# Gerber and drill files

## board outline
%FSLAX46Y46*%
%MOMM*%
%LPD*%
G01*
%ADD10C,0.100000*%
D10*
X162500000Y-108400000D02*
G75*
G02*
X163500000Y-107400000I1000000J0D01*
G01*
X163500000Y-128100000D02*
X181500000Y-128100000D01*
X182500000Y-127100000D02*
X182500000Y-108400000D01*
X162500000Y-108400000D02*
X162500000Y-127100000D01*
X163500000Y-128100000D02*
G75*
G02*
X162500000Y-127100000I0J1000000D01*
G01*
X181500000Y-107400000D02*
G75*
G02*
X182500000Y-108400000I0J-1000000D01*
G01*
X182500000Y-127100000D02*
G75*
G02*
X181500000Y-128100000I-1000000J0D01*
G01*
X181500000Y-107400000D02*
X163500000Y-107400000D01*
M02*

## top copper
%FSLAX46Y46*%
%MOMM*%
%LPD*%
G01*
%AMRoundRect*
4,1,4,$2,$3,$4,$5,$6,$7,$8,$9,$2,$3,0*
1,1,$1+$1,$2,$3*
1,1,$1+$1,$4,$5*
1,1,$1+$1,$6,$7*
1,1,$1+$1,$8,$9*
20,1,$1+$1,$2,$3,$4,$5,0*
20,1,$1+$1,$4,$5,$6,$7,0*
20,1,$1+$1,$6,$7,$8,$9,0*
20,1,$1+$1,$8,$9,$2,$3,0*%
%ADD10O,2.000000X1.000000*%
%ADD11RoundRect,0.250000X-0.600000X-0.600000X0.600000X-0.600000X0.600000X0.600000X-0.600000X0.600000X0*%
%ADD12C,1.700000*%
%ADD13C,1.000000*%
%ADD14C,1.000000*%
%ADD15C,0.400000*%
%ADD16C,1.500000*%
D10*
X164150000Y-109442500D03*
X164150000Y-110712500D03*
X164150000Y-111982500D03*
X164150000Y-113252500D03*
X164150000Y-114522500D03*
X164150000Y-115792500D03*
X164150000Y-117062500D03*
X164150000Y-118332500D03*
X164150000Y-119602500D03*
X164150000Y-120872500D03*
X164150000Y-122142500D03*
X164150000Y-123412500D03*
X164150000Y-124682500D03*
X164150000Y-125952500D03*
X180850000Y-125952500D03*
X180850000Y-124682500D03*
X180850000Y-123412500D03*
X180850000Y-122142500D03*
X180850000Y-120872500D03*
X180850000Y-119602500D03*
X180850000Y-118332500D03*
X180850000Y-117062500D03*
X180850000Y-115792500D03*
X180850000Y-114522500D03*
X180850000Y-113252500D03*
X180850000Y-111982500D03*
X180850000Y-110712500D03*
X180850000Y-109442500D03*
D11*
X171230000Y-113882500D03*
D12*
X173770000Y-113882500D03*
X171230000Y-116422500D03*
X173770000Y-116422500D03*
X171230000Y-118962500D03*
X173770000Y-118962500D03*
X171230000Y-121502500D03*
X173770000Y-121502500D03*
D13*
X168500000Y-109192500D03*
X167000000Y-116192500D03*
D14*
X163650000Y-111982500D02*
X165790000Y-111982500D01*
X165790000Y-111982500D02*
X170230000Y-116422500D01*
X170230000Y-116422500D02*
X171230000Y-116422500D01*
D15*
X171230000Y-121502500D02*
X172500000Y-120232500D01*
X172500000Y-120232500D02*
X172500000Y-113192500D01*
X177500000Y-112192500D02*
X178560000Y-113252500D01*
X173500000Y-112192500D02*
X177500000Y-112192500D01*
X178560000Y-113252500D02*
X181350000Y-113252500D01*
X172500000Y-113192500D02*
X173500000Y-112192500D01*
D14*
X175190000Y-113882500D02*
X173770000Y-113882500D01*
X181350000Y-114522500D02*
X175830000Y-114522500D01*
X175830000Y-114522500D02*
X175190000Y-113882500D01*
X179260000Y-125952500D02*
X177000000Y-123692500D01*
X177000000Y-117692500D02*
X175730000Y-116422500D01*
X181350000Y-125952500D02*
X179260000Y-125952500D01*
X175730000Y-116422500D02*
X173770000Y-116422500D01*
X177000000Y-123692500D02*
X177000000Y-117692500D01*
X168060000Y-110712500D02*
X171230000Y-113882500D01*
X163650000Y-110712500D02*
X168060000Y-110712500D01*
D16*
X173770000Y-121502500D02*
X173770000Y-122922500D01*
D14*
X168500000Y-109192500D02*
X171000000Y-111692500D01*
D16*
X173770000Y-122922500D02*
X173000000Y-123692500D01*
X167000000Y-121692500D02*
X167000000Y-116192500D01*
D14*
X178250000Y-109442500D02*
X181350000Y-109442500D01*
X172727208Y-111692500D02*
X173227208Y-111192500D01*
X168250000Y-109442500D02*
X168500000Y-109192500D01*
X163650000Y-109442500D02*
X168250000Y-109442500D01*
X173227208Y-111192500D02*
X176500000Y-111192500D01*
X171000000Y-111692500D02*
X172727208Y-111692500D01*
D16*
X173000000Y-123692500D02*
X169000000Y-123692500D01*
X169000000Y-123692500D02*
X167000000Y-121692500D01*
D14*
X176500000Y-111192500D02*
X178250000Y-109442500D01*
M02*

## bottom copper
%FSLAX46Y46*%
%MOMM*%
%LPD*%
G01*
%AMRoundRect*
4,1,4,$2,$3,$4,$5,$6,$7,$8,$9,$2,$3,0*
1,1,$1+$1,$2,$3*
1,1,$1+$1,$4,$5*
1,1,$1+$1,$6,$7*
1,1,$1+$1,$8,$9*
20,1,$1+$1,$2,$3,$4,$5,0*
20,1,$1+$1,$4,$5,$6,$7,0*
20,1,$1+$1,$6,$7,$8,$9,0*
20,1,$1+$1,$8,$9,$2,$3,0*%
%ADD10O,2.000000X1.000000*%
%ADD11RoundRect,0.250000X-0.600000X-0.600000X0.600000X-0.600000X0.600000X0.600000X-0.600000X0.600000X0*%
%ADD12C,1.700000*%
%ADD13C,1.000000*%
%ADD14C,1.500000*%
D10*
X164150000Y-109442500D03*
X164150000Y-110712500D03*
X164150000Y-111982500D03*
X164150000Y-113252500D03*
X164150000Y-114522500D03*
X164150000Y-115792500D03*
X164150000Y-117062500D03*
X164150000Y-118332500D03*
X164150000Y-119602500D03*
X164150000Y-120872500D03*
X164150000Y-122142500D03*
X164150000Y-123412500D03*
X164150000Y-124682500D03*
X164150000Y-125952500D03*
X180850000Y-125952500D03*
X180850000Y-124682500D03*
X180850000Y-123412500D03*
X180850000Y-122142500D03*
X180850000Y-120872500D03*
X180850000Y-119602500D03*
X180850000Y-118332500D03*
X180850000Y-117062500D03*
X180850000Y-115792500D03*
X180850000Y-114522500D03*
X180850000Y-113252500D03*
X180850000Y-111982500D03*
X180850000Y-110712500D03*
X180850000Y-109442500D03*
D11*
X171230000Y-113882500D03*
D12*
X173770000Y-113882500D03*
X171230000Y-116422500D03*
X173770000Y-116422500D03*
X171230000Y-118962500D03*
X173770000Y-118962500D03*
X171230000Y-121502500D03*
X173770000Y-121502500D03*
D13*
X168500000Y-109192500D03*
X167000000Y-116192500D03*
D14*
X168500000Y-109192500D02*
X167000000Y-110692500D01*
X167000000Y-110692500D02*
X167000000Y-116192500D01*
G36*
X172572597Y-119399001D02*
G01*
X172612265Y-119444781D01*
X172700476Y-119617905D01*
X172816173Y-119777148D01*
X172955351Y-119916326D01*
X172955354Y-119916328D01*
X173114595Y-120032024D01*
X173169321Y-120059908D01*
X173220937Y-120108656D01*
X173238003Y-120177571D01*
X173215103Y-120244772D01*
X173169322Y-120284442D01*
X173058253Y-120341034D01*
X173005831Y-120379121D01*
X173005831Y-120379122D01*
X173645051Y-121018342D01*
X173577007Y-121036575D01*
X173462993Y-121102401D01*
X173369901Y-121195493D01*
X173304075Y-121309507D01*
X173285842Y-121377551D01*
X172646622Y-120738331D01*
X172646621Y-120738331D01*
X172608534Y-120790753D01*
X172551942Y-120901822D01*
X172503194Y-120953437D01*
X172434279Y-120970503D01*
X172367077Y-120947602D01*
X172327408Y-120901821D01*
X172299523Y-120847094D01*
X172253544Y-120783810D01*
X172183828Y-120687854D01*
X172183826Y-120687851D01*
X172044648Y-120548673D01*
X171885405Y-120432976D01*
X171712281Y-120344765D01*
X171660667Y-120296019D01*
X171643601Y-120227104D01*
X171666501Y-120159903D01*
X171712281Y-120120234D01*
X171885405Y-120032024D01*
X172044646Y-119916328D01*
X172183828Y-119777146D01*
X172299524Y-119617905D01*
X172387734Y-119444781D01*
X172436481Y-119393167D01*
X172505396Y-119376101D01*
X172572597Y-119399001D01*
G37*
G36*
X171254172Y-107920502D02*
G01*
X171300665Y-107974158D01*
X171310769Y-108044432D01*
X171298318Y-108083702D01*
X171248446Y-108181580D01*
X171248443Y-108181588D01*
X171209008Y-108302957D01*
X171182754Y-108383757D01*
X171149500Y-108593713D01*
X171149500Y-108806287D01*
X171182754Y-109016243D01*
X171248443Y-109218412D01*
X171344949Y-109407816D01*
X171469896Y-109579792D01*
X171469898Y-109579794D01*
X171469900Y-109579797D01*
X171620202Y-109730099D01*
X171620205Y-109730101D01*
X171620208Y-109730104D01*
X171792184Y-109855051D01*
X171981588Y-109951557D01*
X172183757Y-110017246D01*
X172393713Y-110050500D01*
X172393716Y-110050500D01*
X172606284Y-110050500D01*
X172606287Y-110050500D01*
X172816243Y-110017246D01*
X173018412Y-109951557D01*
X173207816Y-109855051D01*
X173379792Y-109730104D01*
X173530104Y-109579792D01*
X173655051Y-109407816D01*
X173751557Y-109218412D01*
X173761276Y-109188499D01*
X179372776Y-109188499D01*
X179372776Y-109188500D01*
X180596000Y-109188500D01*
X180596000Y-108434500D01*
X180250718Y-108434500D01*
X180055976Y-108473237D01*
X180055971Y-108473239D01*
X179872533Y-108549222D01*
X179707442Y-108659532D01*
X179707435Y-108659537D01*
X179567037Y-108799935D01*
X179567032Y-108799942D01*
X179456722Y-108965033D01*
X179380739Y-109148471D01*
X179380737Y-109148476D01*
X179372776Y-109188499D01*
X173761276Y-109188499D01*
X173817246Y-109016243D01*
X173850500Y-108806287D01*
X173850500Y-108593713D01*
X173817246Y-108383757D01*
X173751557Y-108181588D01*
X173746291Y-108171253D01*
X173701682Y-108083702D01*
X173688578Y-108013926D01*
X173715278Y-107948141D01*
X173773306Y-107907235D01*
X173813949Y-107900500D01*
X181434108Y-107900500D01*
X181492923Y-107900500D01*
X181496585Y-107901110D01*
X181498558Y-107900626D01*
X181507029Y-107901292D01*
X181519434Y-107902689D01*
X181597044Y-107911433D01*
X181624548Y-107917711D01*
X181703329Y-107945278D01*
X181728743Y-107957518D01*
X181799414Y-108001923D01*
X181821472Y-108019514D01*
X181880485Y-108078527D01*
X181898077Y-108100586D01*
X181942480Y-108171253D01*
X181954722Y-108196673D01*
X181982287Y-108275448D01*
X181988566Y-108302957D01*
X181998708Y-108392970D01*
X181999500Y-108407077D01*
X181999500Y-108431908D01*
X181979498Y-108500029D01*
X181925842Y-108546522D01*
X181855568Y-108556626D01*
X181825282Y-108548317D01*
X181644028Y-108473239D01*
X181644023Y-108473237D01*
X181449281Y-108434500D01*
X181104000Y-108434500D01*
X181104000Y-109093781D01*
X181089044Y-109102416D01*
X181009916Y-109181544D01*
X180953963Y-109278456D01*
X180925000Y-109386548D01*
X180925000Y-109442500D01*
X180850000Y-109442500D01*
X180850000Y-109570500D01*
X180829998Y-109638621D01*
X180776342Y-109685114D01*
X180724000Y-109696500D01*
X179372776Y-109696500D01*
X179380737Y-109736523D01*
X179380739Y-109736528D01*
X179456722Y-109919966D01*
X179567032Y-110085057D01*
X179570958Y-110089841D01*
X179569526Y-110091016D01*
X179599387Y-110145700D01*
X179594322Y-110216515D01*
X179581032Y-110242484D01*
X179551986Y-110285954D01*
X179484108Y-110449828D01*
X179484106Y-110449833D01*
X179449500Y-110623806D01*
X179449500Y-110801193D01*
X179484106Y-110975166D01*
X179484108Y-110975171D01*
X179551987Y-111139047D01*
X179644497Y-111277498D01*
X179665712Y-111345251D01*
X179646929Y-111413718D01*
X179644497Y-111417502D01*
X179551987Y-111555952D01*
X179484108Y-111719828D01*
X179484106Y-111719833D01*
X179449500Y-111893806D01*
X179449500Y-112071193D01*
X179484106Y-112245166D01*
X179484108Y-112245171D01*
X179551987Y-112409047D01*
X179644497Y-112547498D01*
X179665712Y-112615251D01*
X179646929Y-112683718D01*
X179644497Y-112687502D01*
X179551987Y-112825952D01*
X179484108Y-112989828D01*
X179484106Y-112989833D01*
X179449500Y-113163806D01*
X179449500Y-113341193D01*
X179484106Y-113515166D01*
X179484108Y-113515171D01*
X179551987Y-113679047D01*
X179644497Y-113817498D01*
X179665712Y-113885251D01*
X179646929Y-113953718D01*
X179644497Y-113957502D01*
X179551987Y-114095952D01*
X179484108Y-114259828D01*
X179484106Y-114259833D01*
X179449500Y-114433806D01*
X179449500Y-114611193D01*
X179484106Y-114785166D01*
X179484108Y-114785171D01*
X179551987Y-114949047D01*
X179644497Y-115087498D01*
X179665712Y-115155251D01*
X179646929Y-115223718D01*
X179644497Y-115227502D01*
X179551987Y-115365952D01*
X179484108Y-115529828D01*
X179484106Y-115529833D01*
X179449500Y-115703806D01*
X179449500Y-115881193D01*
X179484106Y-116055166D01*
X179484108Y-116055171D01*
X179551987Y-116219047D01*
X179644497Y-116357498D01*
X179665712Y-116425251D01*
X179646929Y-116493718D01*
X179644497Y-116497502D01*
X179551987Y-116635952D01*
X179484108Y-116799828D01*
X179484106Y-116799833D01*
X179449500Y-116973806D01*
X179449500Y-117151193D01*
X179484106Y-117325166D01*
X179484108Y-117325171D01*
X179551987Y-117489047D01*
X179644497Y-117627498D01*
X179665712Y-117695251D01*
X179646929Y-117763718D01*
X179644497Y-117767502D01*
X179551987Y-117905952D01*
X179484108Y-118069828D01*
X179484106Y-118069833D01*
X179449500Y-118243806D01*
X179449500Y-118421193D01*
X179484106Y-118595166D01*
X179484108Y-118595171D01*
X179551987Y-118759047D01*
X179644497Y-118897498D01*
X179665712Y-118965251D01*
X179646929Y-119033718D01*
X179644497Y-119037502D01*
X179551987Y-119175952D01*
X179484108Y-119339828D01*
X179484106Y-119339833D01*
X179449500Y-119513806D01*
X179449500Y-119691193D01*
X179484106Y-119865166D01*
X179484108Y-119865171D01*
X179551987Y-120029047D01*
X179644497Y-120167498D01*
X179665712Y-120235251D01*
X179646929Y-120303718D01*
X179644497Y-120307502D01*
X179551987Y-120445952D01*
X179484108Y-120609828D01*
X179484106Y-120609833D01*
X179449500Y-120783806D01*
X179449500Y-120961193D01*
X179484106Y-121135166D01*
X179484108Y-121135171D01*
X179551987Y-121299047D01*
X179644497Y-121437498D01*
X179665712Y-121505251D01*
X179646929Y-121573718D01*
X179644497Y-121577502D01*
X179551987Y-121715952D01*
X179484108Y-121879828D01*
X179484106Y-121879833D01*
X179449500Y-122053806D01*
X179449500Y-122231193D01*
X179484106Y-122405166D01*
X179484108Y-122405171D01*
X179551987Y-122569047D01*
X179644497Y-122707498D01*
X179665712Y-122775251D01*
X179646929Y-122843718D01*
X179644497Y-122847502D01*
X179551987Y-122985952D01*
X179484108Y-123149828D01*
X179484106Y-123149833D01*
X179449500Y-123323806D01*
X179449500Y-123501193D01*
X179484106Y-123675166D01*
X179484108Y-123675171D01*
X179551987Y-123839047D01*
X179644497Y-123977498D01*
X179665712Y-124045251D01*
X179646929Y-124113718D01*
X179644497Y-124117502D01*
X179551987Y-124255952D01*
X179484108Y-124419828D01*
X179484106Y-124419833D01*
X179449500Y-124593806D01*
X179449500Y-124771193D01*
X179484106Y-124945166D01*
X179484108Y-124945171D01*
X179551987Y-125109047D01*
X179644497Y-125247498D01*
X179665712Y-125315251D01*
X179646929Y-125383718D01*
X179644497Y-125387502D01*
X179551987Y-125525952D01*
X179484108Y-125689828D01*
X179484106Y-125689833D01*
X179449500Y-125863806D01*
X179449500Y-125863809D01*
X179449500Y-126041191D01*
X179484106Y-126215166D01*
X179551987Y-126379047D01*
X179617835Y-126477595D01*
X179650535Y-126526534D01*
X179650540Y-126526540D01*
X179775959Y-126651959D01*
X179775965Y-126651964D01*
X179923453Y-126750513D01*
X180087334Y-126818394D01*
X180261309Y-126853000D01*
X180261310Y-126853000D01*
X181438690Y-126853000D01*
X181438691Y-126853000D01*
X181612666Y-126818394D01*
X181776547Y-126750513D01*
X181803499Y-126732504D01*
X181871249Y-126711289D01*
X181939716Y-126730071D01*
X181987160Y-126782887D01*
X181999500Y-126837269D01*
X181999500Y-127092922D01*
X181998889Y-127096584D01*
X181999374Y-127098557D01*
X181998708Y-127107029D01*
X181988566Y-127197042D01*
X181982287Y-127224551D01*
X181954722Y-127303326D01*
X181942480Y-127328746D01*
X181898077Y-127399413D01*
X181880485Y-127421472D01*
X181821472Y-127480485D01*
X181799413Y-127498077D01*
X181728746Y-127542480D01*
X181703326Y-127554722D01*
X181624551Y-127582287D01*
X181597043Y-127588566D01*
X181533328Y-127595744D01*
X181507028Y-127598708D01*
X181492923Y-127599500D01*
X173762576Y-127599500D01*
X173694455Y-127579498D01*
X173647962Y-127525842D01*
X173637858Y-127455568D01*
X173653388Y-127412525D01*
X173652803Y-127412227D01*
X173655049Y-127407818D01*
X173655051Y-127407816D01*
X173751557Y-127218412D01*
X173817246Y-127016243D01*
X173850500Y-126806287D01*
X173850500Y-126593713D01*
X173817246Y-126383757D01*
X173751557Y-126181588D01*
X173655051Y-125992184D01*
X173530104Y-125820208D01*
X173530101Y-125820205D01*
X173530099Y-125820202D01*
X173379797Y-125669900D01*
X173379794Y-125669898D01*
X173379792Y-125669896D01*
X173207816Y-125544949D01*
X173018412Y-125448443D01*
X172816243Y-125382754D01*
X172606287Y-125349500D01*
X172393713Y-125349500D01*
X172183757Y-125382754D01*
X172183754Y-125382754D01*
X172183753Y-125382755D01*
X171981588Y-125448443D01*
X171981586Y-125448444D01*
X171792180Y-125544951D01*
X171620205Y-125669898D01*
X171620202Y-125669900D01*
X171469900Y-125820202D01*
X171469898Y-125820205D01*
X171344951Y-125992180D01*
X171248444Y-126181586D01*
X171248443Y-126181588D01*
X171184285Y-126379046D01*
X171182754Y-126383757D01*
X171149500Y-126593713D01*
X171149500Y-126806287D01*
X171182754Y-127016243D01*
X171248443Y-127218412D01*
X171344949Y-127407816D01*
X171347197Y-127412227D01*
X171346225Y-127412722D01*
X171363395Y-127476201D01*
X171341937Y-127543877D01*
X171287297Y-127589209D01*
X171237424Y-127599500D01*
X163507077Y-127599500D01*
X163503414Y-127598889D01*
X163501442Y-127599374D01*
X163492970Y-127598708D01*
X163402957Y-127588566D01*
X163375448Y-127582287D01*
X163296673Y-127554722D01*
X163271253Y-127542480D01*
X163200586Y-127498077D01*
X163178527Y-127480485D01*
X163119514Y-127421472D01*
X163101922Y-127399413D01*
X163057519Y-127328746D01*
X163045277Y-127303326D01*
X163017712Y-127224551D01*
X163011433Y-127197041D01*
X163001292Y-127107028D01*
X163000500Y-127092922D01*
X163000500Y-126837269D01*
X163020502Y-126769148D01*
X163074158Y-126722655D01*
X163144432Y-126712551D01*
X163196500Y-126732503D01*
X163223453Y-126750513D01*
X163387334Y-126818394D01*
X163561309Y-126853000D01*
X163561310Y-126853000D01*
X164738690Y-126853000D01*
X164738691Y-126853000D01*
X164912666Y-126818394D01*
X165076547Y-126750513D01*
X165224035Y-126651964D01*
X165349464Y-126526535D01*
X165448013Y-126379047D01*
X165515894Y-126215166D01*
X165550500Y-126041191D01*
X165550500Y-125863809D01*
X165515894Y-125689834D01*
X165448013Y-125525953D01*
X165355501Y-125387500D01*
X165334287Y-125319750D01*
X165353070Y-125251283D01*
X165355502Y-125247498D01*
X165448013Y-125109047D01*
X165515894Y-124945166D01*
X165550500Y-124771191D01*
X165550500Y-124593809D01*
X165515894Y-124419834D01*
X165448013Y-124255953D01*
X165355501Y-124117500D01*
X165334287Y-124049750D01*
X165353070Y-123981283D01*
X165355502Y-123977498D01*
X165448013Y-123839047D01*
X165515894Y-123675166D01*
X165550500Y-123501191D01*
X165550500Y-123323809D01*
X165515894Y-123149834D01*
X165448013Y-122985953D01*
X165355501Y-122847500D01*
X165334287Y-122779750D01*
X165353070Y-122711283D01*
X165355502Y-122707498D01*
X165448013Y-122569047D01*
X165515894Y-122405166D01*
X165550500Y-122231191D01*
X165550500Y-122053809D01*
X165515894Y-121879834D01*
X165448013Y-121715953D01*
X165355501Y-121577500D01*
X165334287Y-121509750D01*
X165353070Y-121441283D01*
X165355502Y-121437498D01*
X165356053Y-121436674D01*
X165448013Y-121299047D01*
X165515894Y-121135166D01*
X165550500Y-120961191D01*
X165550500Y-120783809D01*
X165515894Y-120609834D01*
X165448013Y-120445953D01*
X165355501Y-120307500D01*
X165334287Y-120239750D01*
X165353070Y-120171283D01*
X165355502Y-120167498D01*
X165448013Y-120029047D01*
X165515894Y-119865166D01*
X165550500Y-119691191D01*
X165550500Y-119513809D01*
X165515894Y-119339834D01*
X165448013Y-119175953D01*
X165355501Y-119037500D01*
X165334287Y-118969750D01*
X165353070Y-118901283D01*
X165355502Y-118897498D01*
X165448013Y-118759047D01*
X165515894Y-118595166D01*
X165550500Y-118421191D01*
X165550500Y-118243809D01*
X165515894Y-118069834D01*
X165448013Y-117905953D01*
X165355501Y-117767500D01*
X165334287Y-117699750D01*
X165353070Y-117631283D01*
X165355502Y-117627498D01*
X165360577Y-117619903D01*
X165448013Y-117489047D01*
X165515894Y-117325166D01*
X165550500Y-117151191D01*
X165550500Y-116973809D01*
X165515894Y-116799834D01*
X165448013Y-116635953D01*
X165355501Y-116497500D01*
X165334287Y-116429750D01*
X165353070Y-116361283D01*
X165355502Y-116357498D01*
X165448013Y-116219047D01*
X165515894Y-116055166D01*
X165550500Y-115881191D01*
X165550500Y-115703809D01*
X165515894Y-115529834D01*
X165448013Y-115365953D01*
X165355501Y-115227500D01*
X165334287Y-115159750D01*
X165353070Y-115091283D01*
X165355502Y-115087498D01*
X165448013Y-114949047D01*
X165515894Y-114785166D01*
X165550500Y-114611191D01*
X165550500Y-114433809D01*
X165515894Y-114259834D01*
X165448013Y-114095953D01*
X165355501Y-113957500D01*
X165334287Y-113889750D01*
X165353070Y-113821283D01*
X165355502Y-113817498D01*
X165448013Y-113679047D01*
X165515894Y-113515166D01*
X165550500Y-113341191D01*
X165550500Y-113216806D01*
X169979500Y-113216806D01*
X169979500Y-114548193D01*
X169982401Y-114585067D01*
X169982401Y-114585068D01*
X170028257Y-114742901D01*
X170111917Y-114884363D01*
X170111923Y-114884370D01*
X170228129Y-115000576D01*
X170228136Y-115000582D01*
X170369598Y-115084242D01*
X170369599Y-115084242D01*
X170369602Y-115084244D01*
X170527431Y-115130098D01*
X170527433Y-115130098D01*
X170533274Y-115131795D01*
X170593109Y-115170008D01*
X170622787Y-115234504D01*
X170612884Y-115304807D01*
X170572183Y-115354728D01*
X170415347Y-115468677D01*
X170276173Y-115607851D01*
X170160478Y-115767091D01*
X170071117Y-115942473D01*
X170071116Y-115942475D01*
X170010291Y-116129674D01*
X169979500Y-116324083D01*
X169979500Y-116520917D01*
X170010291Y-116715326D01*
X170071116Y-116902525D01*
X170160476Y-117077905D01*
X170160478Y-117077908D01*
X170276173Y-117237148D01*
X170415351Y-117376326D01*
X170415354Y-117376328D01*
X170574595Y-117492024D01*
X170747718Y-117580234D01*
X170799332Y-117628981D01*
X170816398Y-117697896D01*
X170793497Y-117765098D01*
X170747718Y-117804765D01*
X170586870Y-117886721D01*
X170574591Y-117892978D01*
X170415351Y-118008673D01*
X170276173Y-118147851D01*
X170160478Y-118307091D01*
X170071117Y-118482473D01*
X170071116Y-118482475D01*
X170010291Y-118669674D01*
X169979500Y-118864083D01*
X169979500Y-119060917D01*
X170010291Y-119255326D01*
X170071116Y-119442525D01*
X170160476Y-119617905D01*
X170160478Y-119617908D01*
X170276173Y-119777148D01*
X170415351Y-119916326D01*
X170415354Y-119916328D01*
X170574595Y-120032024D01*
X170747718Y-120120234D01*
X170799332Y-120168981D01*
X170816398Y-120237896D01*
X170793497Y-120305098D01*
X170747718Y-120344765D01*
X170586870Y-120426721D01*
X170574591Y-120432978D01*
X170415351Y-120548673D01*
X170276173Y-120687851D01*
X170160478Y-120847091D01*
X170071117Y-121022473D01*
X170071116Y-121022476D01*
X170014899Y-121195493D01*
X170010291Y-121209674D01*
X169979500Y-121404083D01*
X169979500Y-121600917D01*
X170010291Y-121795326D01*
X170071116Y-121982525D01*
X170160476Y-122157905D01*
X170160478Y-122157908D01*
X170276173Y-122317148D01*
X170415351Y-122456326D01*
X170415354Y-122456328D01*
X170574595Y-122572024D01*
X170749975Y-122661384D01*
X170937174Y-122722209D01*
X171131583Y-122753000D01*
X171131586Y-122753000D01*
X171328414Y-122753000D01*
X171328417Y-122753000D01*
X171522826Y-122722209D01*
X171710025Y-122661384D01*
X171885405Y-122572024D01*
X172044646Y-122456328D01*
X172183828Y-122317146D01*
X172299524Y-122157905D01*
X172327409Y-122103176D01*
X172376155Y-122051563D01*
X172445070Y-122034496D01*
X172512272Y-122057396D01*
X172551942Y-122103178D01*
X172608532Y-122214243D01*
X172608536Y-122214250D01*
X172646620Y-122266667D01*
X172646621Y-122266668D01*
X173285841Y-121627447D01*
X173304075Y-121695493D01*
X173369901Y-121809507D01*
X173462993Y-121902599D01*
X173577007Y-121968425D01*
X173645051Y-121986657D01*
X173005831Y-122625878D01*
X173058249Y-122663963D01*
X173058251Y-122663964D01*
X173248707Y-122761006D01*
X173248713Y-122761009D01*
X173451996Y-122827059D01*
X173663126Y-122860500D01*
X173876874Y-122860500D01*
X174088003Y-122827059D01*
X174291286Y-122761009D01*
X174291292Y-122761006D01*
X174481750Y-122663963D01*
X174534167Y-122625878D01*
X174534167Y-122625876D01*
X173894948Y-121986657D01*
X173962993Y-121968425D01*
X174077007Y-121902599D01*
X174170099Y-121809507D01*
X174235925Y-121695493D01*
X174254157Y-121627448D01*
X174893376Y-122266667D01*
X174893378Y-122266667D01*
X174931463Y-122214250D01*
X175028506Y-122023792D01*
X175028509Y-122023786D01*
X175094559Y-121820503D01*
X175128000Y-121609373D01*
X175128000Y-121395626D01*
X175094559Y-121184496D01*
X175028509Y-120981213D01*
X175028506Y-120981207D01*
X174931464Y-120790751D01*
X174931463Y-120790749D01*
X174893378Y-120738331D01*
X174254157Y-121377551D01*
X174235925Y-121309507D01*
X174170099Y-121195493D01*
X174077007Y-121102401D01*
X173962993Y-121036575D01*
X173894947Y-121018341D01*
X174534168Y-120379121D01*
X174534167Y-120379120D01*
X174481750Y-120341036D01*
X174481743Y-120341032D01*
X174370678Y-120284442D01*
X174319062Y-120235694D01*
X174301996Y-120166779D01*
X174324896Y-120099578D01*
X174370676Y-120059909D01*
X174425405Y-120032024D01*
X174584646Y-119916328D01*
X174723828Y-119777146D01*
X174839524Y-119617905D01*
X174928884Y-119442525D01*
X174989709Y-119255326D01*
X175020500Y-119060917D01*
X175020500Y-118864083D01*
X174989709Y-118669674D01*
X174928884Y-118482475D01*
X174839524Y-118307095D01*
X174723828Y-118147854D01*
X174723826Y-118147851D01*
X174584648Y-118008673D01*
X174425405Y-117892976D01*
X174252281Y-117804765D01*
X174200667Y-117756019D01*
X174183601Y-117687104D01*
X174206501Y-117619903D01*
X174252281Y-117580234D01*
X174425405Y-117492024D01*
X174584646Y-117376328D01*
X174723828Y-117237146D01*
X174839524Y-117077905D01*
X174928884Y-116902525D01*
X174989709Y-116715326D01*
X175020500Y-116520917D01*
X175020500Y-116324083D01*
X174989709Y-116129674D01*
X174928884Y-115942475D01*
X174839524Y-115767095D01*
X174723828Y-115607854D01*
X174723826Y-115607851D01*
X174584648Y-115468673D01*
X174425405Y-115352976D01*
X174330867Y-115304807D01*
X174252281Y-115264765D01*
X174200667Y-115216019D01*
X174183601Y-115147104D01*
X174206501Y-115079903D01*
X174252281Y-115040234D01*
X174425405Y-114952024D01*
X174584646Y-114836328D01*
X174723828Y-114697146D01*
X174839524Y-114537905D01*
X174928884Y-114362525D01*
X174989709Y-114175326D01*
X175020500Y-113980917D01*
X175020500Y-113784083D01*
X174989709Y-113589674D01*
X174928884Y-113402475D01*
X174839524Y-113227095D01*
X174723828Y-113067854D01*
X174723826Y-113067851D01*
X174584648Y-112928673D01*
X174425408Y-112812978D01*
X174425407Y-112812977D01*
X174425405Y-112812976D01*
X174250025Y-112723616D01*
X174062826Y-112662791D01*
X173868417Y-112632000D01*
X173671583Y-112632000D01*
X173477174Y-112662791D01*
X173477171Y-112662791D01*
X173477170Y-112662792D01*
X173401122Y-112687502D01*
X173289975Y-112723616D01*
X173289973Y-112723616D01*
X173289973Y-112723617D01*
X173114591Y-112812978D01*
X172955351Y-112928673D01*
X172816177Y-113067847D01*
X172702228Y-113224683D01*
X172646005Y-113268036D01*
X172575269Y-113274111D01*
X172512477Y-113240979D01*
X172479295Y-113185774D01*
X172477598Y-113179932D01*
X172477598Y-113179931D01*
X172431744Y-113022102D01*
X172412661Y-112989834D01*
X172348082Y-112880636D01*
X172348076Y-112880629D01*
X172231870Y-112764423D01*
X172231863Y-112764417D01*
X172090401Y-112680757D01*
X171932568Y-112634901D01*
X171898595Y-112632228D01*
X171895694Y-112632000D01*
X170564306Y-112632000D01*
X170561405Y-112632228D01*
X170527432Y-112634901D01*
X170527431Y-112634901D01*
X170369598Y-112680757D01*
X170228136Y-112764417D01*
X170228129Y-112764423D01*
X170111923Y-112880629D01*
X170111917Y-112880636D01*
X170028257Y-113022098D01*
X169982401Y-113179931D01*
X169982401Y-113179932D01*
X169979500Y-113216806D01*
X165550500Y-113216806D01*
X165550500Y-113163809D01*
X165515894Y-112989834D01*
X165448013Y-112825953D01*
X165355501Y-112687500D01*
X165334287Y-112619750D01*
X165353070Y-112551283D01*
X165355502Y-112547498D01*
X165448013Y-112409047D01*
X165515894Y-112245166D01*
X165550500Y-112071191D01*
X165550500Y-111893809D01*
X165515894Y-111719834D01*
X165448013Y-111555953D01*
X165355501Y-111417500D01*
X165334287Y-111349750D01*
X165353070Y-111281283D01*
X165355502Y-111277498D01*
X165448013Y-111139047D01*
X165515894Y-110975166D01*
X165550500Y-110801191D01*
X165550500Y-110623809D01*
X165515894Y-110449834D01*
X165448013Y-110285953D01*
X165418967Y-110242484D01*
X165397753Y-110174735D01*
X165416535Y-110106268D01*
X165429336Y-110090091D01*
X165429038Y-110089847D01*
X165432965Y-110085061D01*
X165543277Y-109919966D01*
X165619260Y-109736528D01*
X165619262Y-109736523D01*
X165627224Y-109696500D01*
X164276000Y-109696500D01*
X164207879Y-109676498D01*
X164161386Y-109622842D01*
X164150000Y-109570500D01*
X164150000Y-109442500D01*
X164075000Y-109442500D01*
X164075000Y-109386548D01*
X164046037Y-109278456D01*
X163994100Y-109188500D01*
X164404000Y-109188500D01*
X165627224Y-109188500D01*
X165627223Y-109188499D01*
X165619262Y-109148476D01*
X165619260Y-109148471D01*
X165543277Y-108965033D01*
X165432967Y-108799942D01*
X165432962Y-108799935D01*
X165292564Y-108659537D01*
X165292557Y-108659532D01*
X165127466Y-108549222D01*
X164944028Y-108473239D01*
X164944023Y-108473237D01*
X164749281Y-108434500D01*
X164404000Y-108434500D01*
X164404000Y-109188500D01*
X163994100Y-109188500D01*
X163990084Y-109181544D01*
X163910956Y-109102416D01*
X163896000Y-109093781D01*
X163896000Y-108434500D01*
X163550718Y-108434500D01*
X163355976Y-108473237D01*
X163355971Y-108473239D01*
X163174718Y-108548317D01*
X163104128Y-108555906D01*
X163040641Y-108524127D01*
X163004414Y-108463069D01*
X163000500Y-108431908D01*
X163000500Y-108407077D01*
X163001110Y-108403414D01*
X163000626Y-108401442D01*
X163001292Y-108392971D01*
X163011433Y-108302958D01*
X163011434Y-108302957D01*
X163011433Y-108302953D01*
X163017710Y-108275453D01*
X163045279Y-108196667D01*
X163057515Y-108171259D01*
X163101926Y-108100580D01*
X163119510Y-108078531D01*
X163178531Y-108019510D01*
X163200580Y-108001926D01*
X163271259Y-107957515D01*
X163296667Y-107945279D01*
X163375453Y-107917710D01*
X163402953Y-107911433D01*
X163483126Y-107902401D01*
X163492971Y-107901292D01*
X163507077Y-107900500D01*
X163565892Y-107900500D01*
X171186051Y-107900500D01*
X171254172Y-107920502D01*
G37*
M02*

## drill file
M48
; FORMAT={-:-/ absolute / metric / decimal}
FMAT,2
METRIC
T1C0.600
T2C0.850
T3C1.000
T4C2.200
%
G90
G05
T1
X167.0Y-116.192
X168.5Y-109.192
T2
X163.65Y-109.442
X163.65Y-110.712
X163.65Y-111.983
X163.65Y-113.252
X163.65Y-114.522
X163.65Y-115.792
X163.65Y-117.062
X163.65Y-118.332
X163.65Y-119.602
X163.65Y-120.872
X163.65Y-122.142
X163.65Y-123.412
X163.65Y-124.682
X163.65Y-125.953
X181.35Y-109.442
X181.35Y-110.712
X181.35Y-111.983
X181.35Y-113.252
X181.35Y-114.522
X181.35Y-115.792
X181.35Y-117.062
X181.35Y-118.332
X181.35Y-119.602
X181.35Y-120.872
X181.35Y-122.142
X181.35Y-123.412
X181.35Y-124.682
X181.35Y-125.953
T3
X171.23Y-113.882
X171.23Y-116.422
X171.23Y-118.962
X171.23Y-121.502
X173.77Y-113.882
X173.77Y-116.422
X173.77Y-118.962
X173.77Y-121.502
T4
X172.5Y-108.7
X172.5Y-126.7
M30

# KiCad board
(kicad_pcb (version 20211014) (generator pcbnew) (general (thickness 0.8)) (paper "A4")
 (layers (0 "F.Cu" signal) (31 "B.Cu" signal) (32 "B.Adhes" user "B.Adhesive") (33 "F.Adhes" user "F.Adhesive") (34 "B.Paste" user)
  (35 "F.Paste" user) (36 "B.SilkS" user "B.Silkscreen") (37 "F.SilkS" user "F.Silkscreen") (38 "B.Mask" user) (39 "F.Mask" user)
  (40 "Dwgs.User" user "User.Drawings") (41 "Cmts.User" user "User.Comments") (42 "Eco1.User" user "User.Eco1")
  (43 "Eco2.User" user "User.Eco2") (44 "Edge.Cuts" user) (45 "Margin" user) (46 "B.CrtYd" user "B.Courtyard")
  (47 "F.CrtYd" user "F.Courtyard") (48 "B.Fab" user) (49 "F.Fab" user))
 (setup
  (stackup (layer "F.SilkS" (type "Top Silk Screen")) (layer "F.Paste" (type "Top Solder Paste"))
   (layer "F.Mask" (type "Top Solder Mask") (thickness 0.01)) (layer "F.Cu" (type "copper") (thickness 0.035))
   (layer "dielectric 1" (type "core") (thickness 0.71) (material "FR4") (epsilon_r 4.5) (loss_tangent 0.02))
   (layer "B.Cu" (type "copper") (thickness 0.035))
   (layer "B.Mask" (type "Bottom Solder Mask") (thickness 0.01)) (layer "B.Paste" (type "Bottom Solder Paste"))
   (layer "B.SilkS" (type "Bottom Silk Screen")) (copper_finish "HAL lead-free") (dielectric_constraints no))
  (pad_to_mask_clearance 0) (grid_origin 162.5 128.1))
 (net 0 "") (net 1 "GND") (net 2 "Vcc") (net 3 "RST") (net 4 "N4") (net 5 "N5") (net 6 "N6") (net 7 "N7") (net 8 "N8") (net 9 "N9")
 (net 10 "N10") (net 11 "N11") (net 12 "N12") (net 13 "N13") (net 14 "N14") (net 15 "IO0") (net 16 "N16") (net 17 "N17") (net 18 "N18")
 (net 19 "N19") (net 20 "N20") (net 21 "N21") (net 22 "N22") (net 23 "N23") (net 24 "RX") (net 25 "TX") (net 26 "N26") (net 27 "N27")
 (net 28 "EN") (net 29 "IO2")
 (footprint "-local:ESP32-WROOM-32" (layer "F.Cu") (at 172.5 117.6925)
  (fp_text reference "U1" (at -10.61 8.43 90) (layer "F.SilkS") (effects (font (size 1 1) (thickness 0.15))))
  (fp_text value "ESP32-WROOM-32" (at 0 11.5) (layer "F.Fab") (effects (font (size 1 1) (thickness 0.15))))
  (pad "1" thru_hole oval (at -8.85 -8.25) (size 2 1) (drill 0.85 (offset 0.5 0)) (layers *.Cu *.Mask) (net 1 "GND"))
  (pad "2" thru_hole oval (at -8.85 -6.98) (size 2 1) (drill 0.85 (offset 0.5 0)) (layers *.Cu *.Mask) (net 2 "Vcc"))
  (pad "3" thru_hole oval (at -8.85 -5.71) (size 2 1) (drill 0.85 (offset 0.5 0)) (layers *.Cu *.Mask) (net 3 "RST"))
  (pad "4" thru_hole oval (at -8.85 -4.44) (size 2 1) (drill 0.85 (offset 0.5 0)) (layers *.Cu *.Mask) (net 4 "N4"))
  (pad "5" thru_hole oval (at -8.85 -3.17) (size 2 1) (drill 0.85 (offset 0.5 0)) (layers *.Cu *.Mask) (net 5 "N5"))
  (pad "6" thru_hole oval (at -8.85 -1.9) (size 2 1) (drill 0.85 (offset 0.5 0)) (layers *.Cu *.Mask) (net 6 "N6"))
  (pad "7" thru_hole oval (at -8.85 -0.63) (size 2 1) (drill 0.85 (offset 0.5 0)) (layers *.Cu *.Mask) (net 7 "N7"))
  (pad "8" thru_hole oval (at -8.85 0.64) (size 2 1) (drill 0.85 (offset 0.5 0)) (layers *.Cu *.Mask) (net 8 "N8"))
  (pad "9" thru_hole oval (at -8.85 1.91) (size 2 1) (drill 0.85 (offset 0.5 0)) (layers *.Cu *.Mask) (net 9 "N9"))
  (pad "10" thru_hole oval (at -8.85 3.18) (size 2 1) (drill 0.85 (offset 0.5 0)) (layers *.Cu *.Mask) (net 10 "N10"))
  (pad "11" thru_hole oval (at -8.85 4.45) (size 2 1) (drill 0.85 (offset 0.5 0)) (layers *.Cu *.Mask) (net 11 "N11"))
  (pad "12" thru_hole oval (at -8.85 5.72) (size 2 1) (drill 0.85 (offset 0.5 0)) (layers *.Cu *.Mask) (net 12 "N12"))
  (pad "13" thru_hole oval (at -8.85 6.99) (size 2 1) (drill 0.85 (offset 0.5 0)) (layers *.Cu *.Mask) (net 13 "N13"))
  (pad "14" thru_hole oval (at -8.85 8.26) (size 2 1) (drill 0.85 (offset 0.5 0)) (layers *.Cu *.Mask) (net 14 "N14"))
  (pad "25" thru_hole oval (at 8.85 8.26) (size 2 1) (drill 0.85 (offset -0.5 0)) (layers *.Cu *.Mask) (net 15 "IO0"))
  (pad "26" thru_hole oval (at 8.85 6.99) (size 2 1) (drill 0.85 (offset -0.5 0)) (layers *.Cu *.Mask) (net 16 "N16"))
  (pad "27" thru_hole oval (at 8.85 5.72) (size 2 1) (drill 0.85 (offset -0.5 0)) (layers *.Cu *.Mask) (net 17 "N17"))
  (pad "28" thru_hole oval (at 8.85 4.45) (size 2 1) (drill 0.85 (offset -0.5 0)) (layers *.Cu *.Mask) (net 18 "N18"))
  (pad "29" thru_hole oval (at 8.85 3.18) (size 2 1) (drill 0.85 (offset -0.5 0)) (layers *.Cu *.Mask) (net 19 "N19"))
  (pad "30" thru_hole oval (at 8.85 1.91) (size 2 1) (drill 0.85 (offset -0.5 0)) (layers *.Cu *.Mask) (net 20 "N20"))
  (pad "31" thru_hole oval (at 8.85 0.64) (size 2 1) (drill 0.85 (offset -0.5 0)) (layers *.Cu *.Mask) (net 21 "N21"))
  (pad "32" thru_hole oval (at 8.85 -0.63) (size 2 1) (drill 0.85 (offset -0.5 0)) (layers *.Cu *.Mask) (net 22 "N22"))
  (pad "33" thru_hole oval (at 8.85 -1.9) (size 2 1) (drill 0.85 (offset -0.5 0)) (layers *.Cu *.Mask) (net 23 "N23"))
  (pad "34" thru_hole oval (at 8.85 -3.17) (size 2 1) (drill 0.85 (offset -0.5 0)) (layers *.Cu *.Mask) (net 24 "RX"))
  (pad "35" thru_hole oval (at 8.85 -4.44) (size 2 1) (drill 0.85 (offset -0.5 0)) (layers *.Cu *.Mask) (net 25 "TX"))
  (pad "36" thru_hole oval (at 8.85 -5.71) (size 2 1) (drill 0.85 (offset -0.5 0)) (layers *.Cu *.Mask) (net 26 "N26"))
  (pad "37" thru_hole oval (at 8.85 -6.98) (size 2 1) (drill 0.85 (offset -0.5 0)) (layers *.Cu *.Mask) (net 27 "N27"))
  (pad "38" thru_hole oval (at 8.85 -8.25) (size 2 1) (drill 0.85 (offset -0.5 0)) (layers *.Cu *.Mask) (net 1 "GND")))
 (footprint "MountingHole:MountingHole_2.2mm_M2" (layer "F.Cu") (at 172.5 126.7)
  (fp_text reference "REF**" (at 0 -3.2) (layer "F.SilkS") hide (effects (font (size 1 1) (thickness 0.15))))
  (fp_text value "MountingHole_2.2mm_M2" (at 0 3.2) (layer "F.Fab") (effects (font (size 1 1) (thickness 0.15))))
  (pad "" np_thru_hole circle (at 0 0) (size 2.2 2.2) (drill 2.2) (layers *.Cu *.Mask)))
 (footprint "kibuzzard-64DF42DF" (layer "F.Cu") (at 166.3 109.5 90)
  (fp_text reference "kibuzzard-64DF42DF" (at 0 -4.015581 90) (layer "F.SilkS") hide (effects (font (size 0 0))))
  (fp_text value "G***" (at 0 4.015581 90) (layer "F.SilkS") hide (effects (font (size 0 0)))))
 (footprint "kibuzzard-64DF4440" (layer "F.Cu") (at 178.5 124.9 90)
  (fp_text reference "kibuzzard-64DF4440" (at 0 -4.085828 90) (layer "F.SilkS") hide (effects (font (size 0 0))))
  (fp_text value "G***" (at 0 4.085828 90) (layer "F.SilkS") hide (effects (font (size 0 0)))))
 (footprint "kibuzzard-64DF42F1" (layer "F.Cu") (at 166.3 124.9 90)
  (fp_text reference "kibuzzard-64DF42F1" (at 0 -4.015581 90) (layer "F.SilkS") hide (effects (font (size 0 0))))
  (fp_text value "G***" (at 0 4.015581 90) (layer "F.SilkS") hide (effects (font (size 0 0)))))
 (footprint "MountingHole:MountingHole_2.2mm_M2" (layer "F.Cu") (at 172.5 108.7)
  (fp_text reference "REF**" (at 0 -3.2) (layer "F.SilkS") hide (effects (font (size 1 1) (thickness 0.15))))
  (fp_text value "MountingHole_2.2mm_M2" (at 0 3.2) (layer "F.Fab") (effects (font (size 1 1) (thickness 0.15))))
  (pad "" np_thru_hole circle (at 0 0) (size 2.2 2.2) (drill 2.2) (layers *.Cu *.Mask)))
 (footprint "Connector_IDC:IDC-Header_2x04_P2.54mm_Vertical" (layer "F.Cu") (at 171.23 113.8825)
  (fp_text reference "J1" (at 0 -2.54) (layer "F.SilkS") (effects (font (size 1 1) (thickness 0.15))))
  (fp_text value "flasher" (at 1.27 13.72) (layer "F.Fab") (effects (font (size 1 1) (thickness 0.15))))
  (pad "1" thru_hole roundrect (at 0 0) (size 1.7 1.7) (drill 1) (layers *.Cu *.Mask) (roundrect_rratio 0.147059) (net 2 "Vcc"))
  (pad "2" thru_hole circle (at 2.54 0) (size 1.7 1.7) (drill 1) (layers *.Cu *.Mask) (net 24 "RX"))
  (pad "3" thru_hole circle (at 0 2.54) (size 1.7 1.7) (drill 1) (layers *.Cu *.Mask) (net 3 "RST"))
  (pad "4" thru_hole circle (at 2.54 2.54) (size 1.7 1.7) (drill 1) (layers *.Cu *.Mask) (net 15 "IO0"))
  (pad "5" thru_hole circle (at 0 5.08) (size 1.7 1.7) (drill 1) (layers *.Cu *.Mask) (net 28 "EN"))
  (pad "6" thru_hole circle (at 2.54 5.08) (size 1.7 1.7) (drill 1) (layers *.Cu *.Mask) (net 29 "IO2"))
  (pad "7" thru_hole circle (at 0 7.62) (size 1.7 1.7) (drill 1) (layers *.Cu *.Mask) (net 25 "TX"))
  (pad "8" thru_hole circle (at 2.54 7.62) (size 1.7 1.7) (drill 1) (layers *.Cu *.Mask) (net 1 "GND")))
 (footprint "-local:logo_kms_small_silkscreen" (layer "B.Cu") (at 168.7 124.3 180)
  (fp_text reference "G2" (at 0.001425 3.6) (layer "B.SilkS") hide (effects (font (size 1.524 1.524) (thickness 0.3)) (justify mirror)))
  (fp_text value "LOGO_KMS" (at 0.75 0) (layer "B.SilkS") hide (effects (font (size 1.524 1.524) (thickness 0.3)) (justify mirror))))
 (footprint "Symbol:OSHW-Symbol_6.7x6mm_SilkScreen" (layer "B.Cu") (at 168.7 110.9 180)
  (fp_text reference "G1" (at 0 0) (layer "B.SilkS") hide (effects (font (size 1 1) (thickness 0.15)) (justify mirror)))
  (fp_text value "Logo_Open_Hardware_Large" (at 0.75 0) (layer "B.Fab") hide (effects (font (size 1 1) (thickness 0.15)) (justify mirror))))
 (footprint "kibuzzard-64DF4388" (layer "B.Cu") (at 177.9 117.7 90)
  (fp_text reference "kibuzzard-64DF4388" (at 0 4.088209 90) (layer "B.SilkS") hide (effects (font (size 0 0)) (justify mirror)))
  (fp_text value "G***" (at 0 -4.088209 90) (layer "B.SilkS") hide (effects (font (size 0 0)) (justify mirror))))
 (gr_arc (start 162.5 108.4) (mid 162.792893 107.692893) (end 163.5 107.4) (layer "Edge.Cuts") (width 0.1))
 (gr_line (start 163.5 128.1) (end 181.5 128.1) (layer "Edge.Cuts") (width 0.1))
 (gr_line (start 182.5 127.1) (end 182.5 108.4) (layer "Edge.Cuts") (width 0.1))
 (gr_line (start 162.5 108.4) (end 162.5 127.1) (layer "Edge.Cuts") (width 0.1))
 (gr_arc (start 163.5 128.1) (mid 162.792893 127.807107) (end 162.5 127.1) (layer "Edge.Cuts") (width 0.1))
 (gr_arc (start 181.5 107.4) (mid 182.207107 107.692893) (end 182.5 108.4) (layer "Edge.Cuts") (width 0.1))
 (gr_arc (start 182.5 127.1) (mid 182.207107 127.807107) (end 181.5 128.1) (layer "Edge.Cuts") (width 0.1))
 (gr_line (start 181.5 107.4) (end 163.5 107.4) (layer "Edge.Cuts") (width 0.1))
 (segment (start 163.65 111.9825) (end 165.79 111.9825) (width 1) (layer "F.Cu") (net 3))
 (segment (start 165.79 111.9825) (end 170.23 116.4225) (width 1) (layer "F.Cu") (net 3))
 (segment (start 170.23 116.4225) (end 171.23 116.4225) (width 1) (layer "F.Cu") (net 3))
 (segment (start 171.23 121.5025) (end 172.5 120.2325) (width 0.4) (layer "F.Cu") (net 25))
 (segment (start 172.5 120.2325) (end 172.5 113.1925) (width 0.4) (layer "F.Cu") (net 25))
 (segment (start 177.5 112.1925) (end 178.56 113.2525) (width 0.4) (layer "F.Cu") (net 25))
 (segment (start 173.5 112.1925) (end 177.5 112.1925) (width 0.4) (layer "F.Cu") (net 25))
 (segment (start 178.56 113.2525) (end 181.35 113.2525) (width 0.4) (layer "F.Cu") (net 25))
 (segment (start 172.5 113.1925) (end 173.5 112.1925) (width 0.4) (layer "F.Cu") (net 25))
 (segment (start 175.19 113.8825) (end 173.77 113.8825) (width 1) (layer "F.Cu") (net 24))
 (segment (start 181.35 114.5225) (end 175.83 114.5225) (width 1) (layer "F.Cu") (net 24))
 (segment (start 175.83 114.5225) (end 175.19 113.8825) (width 1) (layer "F.Cu") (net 24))
 (segment (start 179.26 125.9525) (end 177 123.6925) (width 1) (layer "F.Cu") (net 15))
 (segment (start 177 117.6925) (end 175.73 116.4225) (width 1) (layer "F.Cu") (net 15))
 (segment (start 181.35 125.9525) (end 179.26 125.9525) (width 1) (layer "F.Cu") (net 15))
 (segment (start 175.73 116.4225) (end 173.77 116.4225) (width 1) (layer "F.Cu") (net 15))
 (segment (start 177 123.6925) (end 177 117.6925) (width 1) (layer "F.Cu") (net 15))
 (segment (start 168.06 110.7125) (end 171.23 113.8825) (width 1) (layer "F.Cu") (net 2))
 (segment (start 163.65 110.7125) (end 168.06 110.7125) (width 1) (layer "F.Cu") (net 2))
 (segment (start 173.77 121.5025) (end 173.77 122.9225) (width 1.5) (layer "F.Cu") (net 1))
 (segment (start 168.5 109.1925) (end 171 111.6925) (width 1) (layer "F.Cu") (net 1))
 (segment (start 173.77 122.9225) (end 173 123.6925) (width 1.5) (layer "F.Cu") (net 1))
 (segment (start 167 121.6925) (end 167 116.1925) (width 1.5) (layer "F.Cu") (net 1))
 (segment (start 178.25 109.4425) (end 181.35 109.4425) (width 1) (layer "F.Cu") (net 1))
 (segment (start 172.727208 111.6925) (end 173.227208 111.1925) (width 1) (layer "F.Cu") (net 1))
 (segment (start 168.25 109.4425) (end 168.5 109.1925) (width 1) (layer "F.Cu") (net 1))
 (segment (start 163.65 109.4425) (end 168.25 109.4425) (width 1) (layer "F.Cu") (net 1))
 (segment (start 173.227208 111.1925) (end 176.5 111.1925) (width 1) (layer "F.Cu") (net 1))
 (segment (start 171 111.6925) (end 172.727208 111.6925) (width 1) (layer "F.Cu") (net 1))
 (segment (start 173 123.6925) (end 169 123.6925) (width 1.5) (layer "F.Cu") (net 1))
 (segment (start 169 123.6925) (end 167 121.6925) (width 1.5) (layer "F.Cu") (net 1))
 (segment (start 176.5 111.1925) (end 178.25 109.4425) (width 1) (layer "F.Cu") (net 1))
 (via (at 168.5 109.1925) (size 1) (drill 0.6) (layers "F.Cu" "B.Cu") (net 1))
 (via (at 167 116.1925) (size 1) (drill 0.6) (layers "F.Cu" "B.Cu") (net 1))
 (segment (start 168.5 109.1925) (end 167 110.6925) (width 1.5) (layer "B.Cu") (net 1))
 (segment (start 167 110.6925) (end 167 116.1925) (width 1.5) (layer "B.Cu") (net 1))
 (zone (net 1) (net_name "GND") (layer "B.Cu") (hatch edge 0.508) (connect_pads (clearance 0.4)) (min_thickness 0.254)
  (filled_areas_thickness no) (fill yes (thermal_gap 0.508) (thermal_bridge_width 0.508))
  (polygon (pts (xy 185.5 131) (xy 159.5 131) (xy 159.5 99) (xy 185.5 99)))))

